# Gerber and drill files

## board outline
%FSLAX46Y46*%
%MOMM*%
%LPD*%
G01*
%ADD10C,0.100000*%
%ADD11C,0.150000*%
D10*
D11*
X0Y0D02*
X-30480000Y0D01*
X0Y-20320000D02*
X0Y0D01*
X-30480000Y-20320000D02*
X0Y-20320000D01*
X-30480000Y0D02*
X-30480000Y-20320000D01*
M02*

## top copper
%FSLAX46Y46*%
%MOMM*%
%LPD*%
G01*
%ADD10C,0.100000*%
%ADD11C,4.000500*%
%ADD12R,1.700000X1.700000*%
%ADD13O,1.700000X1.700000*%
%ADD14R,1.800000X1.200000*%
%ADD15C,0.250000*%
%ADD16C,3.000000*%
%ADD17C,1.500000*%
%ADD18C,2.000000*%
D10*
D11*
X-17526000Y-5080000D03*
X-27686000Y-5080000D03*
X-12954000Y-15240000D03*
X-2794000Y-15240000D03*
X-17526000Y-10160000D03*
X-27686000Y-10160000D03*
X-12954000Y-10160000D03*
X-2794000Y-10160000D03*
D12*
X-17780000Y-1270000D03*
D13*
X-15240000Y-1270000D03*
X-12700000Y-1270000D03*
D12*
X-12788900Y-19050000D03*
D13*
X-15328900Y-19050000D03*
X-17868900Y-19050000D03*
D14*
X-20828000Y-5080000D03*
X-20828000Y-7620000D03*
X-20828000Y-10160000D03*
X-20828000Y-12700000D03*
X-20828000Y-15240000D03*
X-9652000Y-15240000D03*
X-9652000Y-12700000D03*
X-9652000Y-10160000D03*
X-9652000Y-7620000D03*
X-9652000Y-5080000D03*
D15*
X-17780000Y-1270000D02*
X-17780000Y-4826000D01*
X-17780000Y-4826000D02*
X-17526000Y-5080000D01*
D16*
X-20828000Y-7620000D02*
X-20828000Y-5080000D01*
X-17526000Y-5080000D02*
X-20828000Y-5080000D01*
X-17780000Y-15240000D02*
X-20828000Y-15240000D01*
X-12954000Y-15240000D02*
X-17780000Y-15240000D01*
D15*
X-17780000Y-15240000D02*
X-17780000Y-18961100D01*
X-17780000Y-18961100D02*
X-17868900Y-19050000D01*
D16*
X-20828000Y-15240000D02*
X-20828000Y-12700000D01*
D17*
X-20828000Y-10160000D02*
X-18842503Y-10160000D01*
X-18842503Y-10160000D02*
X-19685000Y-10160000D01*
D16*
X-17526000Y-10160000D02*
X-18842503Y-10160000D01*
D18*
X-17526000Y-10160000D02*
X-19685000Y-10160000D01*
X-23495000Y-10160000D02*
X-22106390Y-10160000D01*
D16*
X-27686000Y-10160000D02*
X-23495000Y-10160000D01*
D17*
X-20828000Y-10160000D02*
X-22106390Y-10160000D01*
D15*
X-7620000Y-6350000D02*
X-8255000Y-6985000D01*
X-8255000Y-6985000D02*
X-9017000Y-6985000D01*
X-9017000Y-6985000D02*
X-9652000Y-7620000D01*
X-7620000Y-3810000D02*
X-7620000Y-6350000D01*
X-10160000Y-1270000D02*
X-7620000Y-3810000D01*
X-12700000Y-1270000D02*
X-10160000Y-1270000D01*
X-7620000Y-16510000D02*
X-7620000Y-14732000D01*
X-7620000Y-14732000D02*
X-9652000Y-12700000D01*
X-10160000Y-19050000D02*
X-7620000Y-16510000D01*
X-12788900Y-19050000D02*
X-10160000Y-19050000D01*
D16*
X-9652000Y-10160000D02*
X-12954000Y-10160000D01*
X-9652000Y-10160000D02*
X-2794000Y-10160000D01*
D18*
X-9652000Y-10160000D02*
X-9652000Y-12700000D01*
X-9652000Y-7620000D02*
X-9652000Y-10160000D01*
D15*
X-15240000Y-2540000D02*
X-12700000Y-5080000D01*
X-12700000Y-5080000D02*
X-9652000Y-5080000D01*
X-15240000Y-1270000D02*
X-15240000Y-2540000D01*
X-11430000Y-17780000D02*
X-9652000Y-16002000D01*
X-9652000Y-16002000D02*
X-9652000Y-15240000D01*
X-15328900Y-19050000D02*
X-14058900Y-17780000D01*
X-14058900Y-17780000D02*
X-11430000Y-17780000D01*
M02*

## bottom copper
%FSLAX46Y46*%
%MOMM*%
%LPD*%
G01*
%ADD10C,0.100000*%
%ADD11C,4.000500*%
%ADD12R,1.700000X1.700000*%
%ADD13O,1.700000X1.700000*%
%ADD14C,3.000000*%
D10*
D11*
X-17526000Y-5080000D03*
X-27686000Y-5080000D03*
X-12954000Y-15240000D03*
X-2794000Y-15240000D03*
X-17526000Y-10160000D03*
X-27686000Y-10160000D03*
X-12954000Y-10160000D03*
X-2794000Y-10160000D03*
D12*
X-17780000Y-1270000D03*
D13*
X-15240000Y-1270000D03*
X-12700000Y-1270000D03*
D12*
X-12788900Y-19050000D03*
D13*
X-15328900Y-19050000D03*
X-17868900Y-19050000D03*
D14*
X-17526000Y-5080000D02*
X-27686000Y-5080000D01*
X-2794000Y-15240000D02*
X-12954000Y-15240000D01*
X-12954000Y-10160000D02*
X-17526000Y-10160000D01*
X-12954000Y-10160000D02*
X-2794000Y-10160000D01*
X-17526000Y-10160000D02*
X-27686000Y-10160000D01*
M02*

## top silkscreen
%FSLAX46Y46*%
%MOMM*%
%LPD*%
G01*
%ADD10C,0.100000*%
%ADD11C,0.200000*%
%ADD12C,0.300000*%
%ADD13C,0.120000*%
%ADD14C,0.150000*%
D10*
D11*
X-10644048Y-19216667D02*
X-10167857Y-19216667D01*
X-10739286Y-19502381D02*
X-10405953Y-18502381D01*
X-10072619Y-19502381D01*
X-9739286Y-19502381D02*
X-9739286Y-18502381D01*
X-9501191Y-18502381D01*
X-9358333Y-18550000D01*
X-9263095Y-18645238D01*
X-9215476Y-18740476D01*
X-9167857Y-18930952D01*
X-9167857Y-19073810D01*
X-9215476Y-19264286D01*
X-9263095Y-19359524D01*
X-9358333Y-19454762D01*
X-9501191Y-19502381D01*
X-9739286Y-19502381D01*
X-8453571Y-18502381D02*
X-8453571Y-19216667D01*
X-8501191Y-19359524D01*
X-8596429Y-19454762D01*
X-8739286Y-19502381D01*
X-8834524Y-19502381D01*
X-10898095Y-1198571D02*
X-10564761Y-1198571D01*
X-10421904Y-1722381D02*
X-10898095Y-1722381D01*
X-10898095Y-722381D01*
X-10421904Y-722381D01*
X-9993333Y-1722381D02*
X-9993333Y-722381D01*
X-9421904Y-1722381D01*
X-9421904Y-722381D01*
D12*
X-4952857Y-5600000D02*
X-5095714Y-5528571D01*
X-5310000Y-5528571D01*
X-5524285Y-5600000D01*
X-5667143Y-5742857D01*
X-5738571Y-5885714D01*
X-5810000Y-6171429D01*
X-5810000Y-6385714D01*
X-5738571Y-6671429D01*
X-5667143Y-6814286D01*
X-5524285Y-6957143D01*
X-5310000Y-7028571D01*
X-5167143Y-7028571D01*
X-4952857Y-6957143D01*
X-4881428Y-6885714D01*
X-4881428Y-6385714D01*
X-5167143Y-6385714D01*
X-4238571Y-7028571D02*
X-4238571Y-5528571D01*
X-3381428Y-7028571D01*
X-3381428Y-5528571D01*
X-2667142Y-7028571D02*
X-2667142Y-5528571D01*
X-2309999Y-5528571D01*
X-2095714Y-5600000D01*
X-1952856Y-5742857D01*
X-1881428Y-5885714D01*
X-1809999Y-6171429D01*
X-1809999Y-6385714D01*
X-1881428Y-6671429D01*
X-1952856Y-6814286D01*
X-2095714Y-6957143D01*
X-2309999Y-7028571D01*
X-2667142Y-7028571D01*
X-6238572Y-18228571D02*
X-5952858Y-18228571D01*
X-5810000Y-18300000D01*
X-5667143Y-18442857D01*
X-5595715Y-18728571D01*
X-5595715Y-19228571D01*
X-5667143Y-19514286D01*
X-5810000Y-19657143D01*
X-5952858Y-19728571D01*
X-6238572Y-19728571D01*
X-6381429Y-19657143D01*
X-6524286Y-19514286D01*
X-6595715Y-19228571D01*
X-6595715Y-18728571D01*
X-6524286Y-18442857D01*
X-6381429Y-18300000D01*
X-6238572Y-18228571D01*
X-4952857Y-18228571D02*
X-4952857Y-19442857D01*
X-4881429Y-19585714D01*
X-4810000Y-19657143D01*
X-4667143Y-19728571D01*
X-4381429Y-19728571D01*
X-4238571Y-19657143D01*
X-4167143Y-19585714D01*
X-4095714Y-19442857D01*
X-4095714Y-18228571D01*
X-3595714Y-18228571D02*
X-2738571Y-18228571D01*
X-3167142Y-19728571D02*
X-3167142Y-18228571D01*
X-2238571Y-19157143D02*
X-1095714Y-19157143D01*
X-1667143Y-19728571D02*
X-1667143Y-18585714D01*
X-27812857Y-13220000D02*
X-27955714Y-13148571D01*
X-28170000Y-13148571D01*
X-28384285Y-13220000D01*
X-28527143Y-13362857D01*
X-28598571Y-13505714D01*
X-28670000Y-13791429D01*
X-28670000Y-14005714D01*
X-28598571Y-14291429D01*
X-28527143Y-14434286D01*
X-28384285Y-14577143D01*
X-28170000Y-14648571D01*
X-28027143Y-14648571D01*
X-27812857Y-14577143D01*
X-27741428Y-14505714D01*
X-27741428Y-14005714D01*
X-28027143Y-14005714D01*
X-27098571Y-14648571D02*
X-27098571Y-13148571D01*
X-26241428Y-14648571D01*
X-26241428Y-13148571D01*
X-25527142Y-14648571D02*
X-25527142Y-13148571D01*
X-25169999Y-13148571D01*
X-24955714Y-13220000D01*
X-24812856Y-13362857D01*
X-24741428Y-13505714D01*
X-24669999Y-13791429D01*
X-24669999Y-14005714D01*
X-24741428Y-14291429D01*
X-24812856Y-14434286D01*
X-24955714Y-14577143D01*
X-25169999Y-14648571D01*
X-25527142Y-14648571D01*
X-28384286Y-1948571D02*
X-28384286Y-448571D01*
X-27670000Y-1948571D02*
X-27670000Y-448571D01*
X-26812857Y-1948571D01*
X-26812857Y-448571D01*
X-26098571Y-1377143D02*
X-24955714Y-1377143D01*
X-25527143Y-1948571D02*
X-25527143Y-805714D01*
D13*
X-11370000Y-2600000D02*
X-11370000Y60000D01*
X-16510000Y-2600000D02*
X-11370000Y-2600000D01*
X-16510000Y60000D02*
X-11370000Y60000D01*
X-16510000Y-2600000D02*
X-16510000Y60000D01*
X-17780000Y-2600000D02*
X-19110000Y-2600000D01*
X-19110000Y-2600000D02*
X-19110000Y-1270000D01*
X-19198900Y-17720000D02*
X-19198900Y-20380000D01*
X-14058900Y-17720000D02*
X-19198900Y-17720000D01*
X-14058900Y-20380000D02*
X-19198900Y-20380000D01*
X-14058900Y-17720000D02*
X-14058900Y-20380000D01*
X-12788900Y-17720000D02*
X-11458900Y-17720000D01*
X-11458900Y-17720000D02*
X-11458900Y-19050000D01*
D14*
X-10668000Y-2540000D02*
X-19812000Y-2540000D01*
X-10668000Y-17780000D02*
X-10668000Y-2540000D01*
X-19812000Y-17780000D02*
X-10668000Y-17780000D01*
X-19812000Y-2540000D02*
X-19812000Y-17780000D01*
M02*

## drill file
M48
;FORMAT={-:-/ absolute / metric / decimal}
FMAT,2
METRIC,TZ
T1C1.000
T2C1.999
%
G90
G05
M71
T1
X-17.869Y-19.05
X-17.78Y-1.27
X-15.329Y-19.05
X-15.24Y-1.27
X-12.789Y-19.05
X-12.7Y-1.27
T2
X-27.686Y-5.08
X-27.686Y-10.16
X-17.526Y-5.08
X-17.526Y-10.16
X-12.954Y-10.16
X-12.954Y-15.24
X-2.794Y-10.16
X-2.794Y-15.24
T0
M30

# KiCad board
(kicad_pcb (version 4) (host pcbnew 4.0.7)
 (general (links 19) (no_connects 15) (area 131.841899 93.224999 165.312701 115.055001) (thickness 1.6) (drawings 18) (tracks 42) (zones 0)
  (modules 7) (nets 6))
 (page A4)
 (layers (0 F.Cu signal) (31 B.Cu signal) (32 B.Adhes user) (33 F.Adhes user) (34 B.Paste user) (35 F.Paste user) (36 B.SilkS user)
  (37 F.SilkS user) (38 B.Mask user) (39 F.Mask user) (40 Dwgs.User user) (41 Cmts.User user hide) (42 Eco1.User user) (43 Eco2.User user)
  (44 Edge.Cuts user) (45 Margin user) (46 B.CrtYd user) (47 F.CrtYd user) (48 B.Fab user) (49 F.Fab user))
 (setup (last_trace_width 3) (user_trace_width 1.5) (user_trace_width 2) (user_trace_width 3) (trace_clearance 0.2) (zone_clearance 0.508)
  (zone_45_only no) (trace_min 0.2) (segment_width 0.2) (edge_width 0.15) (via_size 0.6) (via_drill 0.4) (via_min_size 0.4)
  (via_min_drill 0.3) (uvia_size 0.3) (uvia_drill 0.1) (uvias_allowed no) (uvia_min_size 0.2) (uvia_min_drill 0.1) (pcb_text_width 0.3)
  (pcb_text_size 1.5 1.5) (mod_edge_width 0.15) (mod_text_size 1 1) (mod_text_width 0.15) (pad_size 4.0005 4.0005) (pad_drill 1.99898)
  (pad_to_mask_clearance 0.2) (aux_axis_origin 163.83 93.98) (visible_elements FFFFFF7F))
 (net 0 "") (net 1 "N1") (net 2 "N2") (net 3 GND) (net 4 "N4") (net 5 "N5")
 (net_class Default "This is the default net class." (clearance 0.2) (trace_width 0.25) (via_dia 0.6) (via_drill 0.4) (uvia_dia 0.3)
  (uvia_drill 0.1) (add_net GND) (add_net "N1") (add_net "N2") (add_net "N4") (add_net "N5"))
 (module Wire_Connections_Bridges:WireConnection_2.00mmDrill (layer F.Cu) (at 146.304 99.06 180)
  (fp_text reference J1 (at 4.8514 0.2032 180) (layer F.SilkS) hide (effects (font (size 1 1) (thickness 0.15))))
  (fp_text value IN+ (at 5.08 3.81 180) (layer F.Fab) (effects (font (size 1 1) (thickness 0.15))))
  (pad 1 thru_hole circle (at 0 0 180) (size 4.0005 4.0005) (drill 1.99898) (layers *.Cu B.Mask) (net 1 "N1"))
  (pad 2 thru_hole circle (at 10.16 0 180) (size 4.0005 4.0005) (drill 1.99898) (layers *.Cu *.Mask) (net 1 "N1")))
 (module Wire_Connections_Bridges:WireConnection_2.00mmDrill (layer F.Cu) (at 150.876 109.22)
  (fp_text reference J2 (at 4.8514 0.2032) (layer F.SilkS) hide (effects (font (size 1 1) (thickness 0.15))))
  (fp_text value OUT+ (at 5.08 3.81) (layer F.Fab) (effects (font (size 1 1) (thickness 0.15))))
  (pad 1 thru_hole circle (at 0 0) (size 4.0005 4.0005) (drill 1.99898) (layers *.Cu B.Mask) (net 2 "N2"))
  (pad 2 thru_hole circle (at 10.16 0) (size 4.0005 4.0005) (drill 1.99898) (layers *.Cu *.Mask) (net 2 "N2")))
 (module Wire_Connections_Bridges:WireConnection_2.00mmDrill (layer F.Cu) (at 146.304 104.14 180)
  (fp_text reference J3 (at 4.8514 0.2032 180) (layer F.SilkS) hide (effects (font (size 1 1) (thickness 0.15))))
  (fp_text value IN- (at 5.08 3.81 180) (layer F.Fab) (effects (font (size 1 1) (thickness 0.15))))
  (pad 1 thru_hole circle (at 0 0 180) (size 4.0005 4.0005) (drill 1.99898) (layers *.Cu B.Mask) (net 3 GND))
  (pad 2 thru_hole circle (at 10.16 0 180) (size 4.0005 4.0005) (drill 1.99898) (layers *.Cu *.Mask) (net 3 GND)))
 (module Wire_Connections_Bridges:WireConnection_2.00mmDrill (layer F.Cu) (at 150.876 104.14)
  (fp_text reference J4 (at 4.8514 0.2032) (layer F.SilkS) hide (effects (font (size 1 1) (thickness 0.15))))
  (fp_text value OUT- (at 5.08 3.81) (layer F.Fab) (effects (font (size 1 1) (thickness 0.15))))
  (pad 1 thru_hole circle (at 0 0) (size 4.0005 4.0005) (drill 1.99898) (layers *.Cu B.Mask) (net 3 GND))
  (pad 2 thru_hole circle (at 10.16 0) (size 4.0005 4.0005) (drill 1.99898) (layers *.Cu *.Mask) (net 3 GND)))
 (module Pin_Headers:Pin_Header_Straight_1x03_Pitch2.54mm (layer F.Cu) (at 146.05 95.25 90)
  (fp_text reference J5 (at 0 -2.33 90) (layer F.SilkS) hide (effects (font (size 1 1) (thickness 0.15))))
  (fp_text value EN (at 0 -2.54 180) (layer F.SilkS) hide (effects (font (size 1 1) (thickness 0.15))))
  (fp_line (start -1.33 6.41) (end 1.33 6.41) (layer F.SilkS) (width 0.12))
  (fp_line (start -1.33 1.27) (end -1.33 6.41) (layer F.SilkS) (width 0.12))
  (fp_line (start 1.33 1.27) (end 1.33 6.41) (layer F.SilkS) (width 0.12))
  (fp_line (start -1.33 1.27) (end 1.33 1.27) (layer F.SilkS) (width 0.12))
  (fp_line (start -1.33 0) (end -1.33 -1.33) (layer F.SilkS) (width 0.12))
  (fp_line (start -1.33 -1.33) (end 0 -1.33) (layer F.SilkS) (width 0.12))
  (pad 1 thru_hole rect (at 0 0 90) (size 1.7 1.7) (drill 1) (layers *.Cu *.Mask) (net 1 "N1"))
  (pad 2 thru_hole oval (at 0 2.54 90) (size 1.7 1.7) (drill 1) (layers *.Cu *.Mask) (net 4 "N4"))
  (pad 3 thru_hole oval (at 0 5.08 90) (size 1.7 1.7) (drill 1) (layers *.Cu *.Mask) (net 3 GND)))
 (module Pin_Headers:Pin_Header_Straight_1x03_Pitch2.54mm (layer F.Cu) (at 151.0411 113.03 270)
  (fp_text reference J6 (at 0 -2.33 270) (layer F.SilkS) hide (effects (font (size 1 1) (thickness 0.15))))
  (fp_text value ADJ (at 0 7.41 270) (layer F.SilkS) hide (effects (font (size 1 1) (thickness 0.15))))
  (fp_line (start -1.33 6.41) (end 1.33 6.41) (layer F.SilkS) (width 0.12))
  (fp_line (start -1.33 1.27) (end -1.33 6.41) (layer F.SilkS) (width 0.12))
  (fp_line (start 1.33 1.27) (end 1.33 6.41) (layer F.SilkS) (width 0.12))
  (fp_line (start -1.33 1.27) (end 1.33 1.27) (layer F.SilkS) (width 0.12))
  (fp_line (start -1.33 0) (end -1.33 -1.33) (layer F.SilkS) (width 0.12))
  (fp_line (start -1.33 -1.33) (end 0 -1.33) (layer F.SilkS) (width 0.12))
  (pad 1 thru_hole rect (at 0 0 270) (size 1.7 1.7) (drill 1) (layers *.Cu *.Mask) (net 3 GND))
  (pad 2 thru_hole oval (at 0 2.54 270) (size 1.7 1.7) (drill 1) (layers *.Cu *.Mask) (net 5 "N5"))
  (pad 3 thru_hole oval (at 0 5.08 270) (size 1.7 1.7) (drill 1) (layers *.Cu *.Mask) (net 2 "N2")))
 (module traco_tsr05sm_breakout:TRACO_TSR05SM (layer F.Cu) (at 148.59 104.14)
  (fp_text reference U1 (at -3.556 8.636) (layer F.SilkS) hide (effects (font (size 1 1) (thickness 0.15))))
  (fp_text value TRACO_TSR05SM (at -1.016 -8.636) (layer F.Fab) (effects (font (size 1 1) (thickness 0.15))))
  (fp_line (start 4.572 -7.62) (end -4.572 -7.62) (layer F.SilkS) (width 0.15))
  (fp_line (start 4.572 7.62) (end 4.572 -7.62) (layer F.SilkS) (width 0.15))
  (fp_line (start -4.572 7.62) (end 4.572 7.62) (layer F.SilkS) (width 0.15))
  (fp_line (start -4.572 -7.62) (end -4.572 7.62) (layer F.SilkS) (width 0.15))
  (pad 1 smd rect (at -5.588 -5.08) (size 1.8 1.2) (layers F.Cu F.Paste F.Mask) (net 1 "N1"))
  (pad 2 smd rect (at -5.588 -2.54) (size 1.8 1.2) (layers F.Cu F.Paste F.Mask) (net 1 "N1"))
  (pad 3 smd rect (at -5.588 0) (size 1.8 1.2) (layers F.Cu F.Paste F.Mask) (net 3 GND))
  (pad 4 smd rect (at -5.588 2.54) (size 1.8 1.2) (layers F.Cu F.Paste F.Mask) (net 2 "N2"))
  (pad 5 smd rect (at -5.588 5.08) (size 1.8 1.2) (layers F.Cu F.Paste F.Mask) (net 2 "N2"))
  (pad 6 smd rect (at 5.588 5.08) (size 1.8 1.2) (layers F.Cu F.Paste F.Mask) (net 5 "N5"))
  (pad 7 smd rect (at 5.588 2.54) (size 1.8 1.2) (layers F.Cu F.Paste F.Mask) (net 3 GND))
  (pad 8 smd rect (at 5.588 0) (size 1.8 1.2) (layers F.Cu F.Paste F.Mask) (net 3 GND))
  (pad 9 smd rect (at 5.588 -2.54) (size 1.8 1.2) (layers F.Cu F.Paste F.Mask) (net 3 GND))
  (pad 10 smd rect (at 5.588 -5.08) (size 1.8 1.2) (layers F.Cu F.Paste F.Mask) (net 4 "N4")))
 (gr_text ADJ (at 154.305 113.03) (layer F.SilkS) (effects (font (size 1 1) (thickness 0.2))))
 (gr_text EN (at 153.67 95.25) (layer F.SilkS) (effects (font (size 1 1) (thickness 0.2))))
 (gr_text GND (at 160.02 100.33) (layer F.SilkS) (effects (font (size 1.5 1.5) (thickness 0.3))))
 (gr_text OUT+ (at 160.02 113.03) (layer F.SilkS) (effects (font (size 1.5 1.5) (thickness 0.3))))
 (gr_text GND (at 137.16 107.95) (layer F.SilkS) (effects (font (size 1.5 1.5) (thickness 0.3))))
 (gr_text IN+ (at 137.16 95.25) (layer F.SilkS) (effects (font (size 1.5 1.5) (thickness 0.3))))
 (gr_line (start 163.83 93.98) (end 133.35 93.98) (layer Edge.Cuts) (width 0.15))
 (gr_line (start 163.83 114.3) (end 163.83 93.98) (layer Edge.Cuts) (width 0.15))
 (gr_line (start 133.35 114.3) (end 163.83 114.3) (layer Edge.Cuts) (width 0.15))
 (gr_line (start 133.35 93.98) (end 133.35 114.3) (layer Edge.Cuts) (width 0.15))
 (segment (start 146.05 95.25) (end 146.05 98.806) (width 0.25) (layer F.Cu) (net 1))
 (segment (start 146.05 98.806) (end 146.304 99.06) (width 0.25) (layer F.Cu) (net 1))
 (segment (start 143.002 101.6) (end 143.002 99.06) (width 3) (layer F.Cu) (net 1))
 (segment (start 146.304 99.06) (end 143.002 99.06) (width 3) (layer F.Cu) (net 1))
 (segment (start 146.304 99.06) (end 136.144 99.06) (width 3) (layer B.Cu) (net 1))
 (segment (start 146.05 109.22) (end 143.002 109.22) (width 3) (layer F.Cu) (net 2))
 (segment (start 150.876 109.22) (end 146.05 109.22) (width 3) (layer F.Cu) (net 2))
 (segment (start 146.05 109.22) (end 146.05 112.9411) (width 0.25) (layer F.Cu) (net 2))
 (segment (start 146.05 112.9411) (end 145.9611 113.03) (width 0.25) (layer F.Cu) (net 2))
 (segment (start 143.002 109.22) (end 143.002 106.68) (width 3) (layer F.Cu) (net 2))
 (segment (start 161.036 109.22) (end 150.876 109.22) (width 3) (layer B.Cu) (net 2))
 (segment (start 150.876 104.14) (end 146.304 104.14) (width 3) (layer B.Cu) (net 3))
 (segment (start 143.002 104.14) (end 144.987497 104.14) (width 1.5) (layer F.Cu) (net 3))
 (segment (start 144.987497 104.14) (end 144.145 104.14) (width 1.5) (layer F.Cu) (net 3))
 (segment (start 146.304 104.14) (end 144.987497 104.14) (width 3) (layer F.Cu) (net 3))
 (segment (start 146.304 104.14) (end 144.145 104.14) (width 2) (layer F.Cu) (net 3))
 (segment (start 140.335 104.14) (end 141.72361 104.14) (width 2) (layer F.Cu) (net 3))
 (segment (start 136.144 104.14) (end 140.335 104.14) (width 3) (layer F.Cu) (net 3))
 (segment (start 143.002 104.14) (end 141.72361 104.14) (width 1.5) (layer F.Cu) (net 3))
 (segment (start 156.21 100.33) (end 155.575 100.965) (width 0.25) (layer F.Cu) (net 3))
 (segment (start 155.575 100.965) (end 154.813 100.965) (width 0.25) (layer F.Cu) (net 3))
 (segment (start 154.813 100.965) (end 154.178 101.6) (width 0.25) (layer F.Cu) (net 3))
 (segment (start 156.21 97.79) (end 156.21 100.33) (width 0.25) (layer F.Cu) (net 3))
 (segment (start 153.67 95.25) (end 156.21 97.79) (width 0.25) (layer F.Cu) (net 3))
 (segment (start 151.13 95.25) (end 153.67 95.25) (width 0.25) (layer F.Cu) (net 3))
 (segment (start 156.21 110.49) (end 156.21 108.712) (width 0.25) (layer F.Cu) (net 3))
 (segment (start 156.21 108.712) (end 154.178 106.68) (width 0.25) (layer F.Cu) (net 3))
 (segment (start 153.67 113.03) (end 156.21 110.49) (width 0.25) (layer F.Cu) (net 3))
 (segment (start 151.0411 113.03) (end 153.67 113.03) (width 0.25) (layer F.Cu) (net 3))
 (segment (start 154.178 104.14) (end 150.876 104.14) (width 3) (layer F.Cu) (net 3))
 (segment (start 154.178 104.14) (end 161.036 104.14) (width 3) (layer F.Cu) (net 3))
 (segment (start 154.178 104.14) (end 154.178 106.68) (width 2) (layer F.Cu) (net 3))
 (segment (start 154.178 101.6) (end 154.178 104.14) (width 2) (layer F.Cu) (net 3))
 (segment (start 150.876 104.14) (end 161.036 104.14) (width 3) (layer B.Cu) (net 3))
 (segment (start 146.304 104.14) (end 136.144 104.14) (width 3) (layer B.Cu) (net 3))
 (segment (start 148.59 96.52) (end 151.13 99.06) (width 0.25) (layer F.Cu) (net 4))
 (segment (start 151.13 99.06) (end 154.178 99.06) (width 0.25) (layer F.Cu) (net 4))
 (segment (start 148.59 95.25) (end 148.59 96.52) (width 0.25) (layer F.Cu) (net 4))
 (segment (start 152.4 111.76) (end 154.178 109.982) (width 0.25) (layer F.Cu) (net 5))
 (segment (start 154.178 109.982) (end 154.178 109.22) (width 0.25) (layer F.Cu) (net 5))
 (segment (start 148.5011 113.03) (end 149.7711 111.76) (width 0.25) (layer F.Cu) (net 5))
 (segment (start 149.7711 111.76) (end 152.4 111.76) (width 0.25) (layer F.Cu) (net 5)))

